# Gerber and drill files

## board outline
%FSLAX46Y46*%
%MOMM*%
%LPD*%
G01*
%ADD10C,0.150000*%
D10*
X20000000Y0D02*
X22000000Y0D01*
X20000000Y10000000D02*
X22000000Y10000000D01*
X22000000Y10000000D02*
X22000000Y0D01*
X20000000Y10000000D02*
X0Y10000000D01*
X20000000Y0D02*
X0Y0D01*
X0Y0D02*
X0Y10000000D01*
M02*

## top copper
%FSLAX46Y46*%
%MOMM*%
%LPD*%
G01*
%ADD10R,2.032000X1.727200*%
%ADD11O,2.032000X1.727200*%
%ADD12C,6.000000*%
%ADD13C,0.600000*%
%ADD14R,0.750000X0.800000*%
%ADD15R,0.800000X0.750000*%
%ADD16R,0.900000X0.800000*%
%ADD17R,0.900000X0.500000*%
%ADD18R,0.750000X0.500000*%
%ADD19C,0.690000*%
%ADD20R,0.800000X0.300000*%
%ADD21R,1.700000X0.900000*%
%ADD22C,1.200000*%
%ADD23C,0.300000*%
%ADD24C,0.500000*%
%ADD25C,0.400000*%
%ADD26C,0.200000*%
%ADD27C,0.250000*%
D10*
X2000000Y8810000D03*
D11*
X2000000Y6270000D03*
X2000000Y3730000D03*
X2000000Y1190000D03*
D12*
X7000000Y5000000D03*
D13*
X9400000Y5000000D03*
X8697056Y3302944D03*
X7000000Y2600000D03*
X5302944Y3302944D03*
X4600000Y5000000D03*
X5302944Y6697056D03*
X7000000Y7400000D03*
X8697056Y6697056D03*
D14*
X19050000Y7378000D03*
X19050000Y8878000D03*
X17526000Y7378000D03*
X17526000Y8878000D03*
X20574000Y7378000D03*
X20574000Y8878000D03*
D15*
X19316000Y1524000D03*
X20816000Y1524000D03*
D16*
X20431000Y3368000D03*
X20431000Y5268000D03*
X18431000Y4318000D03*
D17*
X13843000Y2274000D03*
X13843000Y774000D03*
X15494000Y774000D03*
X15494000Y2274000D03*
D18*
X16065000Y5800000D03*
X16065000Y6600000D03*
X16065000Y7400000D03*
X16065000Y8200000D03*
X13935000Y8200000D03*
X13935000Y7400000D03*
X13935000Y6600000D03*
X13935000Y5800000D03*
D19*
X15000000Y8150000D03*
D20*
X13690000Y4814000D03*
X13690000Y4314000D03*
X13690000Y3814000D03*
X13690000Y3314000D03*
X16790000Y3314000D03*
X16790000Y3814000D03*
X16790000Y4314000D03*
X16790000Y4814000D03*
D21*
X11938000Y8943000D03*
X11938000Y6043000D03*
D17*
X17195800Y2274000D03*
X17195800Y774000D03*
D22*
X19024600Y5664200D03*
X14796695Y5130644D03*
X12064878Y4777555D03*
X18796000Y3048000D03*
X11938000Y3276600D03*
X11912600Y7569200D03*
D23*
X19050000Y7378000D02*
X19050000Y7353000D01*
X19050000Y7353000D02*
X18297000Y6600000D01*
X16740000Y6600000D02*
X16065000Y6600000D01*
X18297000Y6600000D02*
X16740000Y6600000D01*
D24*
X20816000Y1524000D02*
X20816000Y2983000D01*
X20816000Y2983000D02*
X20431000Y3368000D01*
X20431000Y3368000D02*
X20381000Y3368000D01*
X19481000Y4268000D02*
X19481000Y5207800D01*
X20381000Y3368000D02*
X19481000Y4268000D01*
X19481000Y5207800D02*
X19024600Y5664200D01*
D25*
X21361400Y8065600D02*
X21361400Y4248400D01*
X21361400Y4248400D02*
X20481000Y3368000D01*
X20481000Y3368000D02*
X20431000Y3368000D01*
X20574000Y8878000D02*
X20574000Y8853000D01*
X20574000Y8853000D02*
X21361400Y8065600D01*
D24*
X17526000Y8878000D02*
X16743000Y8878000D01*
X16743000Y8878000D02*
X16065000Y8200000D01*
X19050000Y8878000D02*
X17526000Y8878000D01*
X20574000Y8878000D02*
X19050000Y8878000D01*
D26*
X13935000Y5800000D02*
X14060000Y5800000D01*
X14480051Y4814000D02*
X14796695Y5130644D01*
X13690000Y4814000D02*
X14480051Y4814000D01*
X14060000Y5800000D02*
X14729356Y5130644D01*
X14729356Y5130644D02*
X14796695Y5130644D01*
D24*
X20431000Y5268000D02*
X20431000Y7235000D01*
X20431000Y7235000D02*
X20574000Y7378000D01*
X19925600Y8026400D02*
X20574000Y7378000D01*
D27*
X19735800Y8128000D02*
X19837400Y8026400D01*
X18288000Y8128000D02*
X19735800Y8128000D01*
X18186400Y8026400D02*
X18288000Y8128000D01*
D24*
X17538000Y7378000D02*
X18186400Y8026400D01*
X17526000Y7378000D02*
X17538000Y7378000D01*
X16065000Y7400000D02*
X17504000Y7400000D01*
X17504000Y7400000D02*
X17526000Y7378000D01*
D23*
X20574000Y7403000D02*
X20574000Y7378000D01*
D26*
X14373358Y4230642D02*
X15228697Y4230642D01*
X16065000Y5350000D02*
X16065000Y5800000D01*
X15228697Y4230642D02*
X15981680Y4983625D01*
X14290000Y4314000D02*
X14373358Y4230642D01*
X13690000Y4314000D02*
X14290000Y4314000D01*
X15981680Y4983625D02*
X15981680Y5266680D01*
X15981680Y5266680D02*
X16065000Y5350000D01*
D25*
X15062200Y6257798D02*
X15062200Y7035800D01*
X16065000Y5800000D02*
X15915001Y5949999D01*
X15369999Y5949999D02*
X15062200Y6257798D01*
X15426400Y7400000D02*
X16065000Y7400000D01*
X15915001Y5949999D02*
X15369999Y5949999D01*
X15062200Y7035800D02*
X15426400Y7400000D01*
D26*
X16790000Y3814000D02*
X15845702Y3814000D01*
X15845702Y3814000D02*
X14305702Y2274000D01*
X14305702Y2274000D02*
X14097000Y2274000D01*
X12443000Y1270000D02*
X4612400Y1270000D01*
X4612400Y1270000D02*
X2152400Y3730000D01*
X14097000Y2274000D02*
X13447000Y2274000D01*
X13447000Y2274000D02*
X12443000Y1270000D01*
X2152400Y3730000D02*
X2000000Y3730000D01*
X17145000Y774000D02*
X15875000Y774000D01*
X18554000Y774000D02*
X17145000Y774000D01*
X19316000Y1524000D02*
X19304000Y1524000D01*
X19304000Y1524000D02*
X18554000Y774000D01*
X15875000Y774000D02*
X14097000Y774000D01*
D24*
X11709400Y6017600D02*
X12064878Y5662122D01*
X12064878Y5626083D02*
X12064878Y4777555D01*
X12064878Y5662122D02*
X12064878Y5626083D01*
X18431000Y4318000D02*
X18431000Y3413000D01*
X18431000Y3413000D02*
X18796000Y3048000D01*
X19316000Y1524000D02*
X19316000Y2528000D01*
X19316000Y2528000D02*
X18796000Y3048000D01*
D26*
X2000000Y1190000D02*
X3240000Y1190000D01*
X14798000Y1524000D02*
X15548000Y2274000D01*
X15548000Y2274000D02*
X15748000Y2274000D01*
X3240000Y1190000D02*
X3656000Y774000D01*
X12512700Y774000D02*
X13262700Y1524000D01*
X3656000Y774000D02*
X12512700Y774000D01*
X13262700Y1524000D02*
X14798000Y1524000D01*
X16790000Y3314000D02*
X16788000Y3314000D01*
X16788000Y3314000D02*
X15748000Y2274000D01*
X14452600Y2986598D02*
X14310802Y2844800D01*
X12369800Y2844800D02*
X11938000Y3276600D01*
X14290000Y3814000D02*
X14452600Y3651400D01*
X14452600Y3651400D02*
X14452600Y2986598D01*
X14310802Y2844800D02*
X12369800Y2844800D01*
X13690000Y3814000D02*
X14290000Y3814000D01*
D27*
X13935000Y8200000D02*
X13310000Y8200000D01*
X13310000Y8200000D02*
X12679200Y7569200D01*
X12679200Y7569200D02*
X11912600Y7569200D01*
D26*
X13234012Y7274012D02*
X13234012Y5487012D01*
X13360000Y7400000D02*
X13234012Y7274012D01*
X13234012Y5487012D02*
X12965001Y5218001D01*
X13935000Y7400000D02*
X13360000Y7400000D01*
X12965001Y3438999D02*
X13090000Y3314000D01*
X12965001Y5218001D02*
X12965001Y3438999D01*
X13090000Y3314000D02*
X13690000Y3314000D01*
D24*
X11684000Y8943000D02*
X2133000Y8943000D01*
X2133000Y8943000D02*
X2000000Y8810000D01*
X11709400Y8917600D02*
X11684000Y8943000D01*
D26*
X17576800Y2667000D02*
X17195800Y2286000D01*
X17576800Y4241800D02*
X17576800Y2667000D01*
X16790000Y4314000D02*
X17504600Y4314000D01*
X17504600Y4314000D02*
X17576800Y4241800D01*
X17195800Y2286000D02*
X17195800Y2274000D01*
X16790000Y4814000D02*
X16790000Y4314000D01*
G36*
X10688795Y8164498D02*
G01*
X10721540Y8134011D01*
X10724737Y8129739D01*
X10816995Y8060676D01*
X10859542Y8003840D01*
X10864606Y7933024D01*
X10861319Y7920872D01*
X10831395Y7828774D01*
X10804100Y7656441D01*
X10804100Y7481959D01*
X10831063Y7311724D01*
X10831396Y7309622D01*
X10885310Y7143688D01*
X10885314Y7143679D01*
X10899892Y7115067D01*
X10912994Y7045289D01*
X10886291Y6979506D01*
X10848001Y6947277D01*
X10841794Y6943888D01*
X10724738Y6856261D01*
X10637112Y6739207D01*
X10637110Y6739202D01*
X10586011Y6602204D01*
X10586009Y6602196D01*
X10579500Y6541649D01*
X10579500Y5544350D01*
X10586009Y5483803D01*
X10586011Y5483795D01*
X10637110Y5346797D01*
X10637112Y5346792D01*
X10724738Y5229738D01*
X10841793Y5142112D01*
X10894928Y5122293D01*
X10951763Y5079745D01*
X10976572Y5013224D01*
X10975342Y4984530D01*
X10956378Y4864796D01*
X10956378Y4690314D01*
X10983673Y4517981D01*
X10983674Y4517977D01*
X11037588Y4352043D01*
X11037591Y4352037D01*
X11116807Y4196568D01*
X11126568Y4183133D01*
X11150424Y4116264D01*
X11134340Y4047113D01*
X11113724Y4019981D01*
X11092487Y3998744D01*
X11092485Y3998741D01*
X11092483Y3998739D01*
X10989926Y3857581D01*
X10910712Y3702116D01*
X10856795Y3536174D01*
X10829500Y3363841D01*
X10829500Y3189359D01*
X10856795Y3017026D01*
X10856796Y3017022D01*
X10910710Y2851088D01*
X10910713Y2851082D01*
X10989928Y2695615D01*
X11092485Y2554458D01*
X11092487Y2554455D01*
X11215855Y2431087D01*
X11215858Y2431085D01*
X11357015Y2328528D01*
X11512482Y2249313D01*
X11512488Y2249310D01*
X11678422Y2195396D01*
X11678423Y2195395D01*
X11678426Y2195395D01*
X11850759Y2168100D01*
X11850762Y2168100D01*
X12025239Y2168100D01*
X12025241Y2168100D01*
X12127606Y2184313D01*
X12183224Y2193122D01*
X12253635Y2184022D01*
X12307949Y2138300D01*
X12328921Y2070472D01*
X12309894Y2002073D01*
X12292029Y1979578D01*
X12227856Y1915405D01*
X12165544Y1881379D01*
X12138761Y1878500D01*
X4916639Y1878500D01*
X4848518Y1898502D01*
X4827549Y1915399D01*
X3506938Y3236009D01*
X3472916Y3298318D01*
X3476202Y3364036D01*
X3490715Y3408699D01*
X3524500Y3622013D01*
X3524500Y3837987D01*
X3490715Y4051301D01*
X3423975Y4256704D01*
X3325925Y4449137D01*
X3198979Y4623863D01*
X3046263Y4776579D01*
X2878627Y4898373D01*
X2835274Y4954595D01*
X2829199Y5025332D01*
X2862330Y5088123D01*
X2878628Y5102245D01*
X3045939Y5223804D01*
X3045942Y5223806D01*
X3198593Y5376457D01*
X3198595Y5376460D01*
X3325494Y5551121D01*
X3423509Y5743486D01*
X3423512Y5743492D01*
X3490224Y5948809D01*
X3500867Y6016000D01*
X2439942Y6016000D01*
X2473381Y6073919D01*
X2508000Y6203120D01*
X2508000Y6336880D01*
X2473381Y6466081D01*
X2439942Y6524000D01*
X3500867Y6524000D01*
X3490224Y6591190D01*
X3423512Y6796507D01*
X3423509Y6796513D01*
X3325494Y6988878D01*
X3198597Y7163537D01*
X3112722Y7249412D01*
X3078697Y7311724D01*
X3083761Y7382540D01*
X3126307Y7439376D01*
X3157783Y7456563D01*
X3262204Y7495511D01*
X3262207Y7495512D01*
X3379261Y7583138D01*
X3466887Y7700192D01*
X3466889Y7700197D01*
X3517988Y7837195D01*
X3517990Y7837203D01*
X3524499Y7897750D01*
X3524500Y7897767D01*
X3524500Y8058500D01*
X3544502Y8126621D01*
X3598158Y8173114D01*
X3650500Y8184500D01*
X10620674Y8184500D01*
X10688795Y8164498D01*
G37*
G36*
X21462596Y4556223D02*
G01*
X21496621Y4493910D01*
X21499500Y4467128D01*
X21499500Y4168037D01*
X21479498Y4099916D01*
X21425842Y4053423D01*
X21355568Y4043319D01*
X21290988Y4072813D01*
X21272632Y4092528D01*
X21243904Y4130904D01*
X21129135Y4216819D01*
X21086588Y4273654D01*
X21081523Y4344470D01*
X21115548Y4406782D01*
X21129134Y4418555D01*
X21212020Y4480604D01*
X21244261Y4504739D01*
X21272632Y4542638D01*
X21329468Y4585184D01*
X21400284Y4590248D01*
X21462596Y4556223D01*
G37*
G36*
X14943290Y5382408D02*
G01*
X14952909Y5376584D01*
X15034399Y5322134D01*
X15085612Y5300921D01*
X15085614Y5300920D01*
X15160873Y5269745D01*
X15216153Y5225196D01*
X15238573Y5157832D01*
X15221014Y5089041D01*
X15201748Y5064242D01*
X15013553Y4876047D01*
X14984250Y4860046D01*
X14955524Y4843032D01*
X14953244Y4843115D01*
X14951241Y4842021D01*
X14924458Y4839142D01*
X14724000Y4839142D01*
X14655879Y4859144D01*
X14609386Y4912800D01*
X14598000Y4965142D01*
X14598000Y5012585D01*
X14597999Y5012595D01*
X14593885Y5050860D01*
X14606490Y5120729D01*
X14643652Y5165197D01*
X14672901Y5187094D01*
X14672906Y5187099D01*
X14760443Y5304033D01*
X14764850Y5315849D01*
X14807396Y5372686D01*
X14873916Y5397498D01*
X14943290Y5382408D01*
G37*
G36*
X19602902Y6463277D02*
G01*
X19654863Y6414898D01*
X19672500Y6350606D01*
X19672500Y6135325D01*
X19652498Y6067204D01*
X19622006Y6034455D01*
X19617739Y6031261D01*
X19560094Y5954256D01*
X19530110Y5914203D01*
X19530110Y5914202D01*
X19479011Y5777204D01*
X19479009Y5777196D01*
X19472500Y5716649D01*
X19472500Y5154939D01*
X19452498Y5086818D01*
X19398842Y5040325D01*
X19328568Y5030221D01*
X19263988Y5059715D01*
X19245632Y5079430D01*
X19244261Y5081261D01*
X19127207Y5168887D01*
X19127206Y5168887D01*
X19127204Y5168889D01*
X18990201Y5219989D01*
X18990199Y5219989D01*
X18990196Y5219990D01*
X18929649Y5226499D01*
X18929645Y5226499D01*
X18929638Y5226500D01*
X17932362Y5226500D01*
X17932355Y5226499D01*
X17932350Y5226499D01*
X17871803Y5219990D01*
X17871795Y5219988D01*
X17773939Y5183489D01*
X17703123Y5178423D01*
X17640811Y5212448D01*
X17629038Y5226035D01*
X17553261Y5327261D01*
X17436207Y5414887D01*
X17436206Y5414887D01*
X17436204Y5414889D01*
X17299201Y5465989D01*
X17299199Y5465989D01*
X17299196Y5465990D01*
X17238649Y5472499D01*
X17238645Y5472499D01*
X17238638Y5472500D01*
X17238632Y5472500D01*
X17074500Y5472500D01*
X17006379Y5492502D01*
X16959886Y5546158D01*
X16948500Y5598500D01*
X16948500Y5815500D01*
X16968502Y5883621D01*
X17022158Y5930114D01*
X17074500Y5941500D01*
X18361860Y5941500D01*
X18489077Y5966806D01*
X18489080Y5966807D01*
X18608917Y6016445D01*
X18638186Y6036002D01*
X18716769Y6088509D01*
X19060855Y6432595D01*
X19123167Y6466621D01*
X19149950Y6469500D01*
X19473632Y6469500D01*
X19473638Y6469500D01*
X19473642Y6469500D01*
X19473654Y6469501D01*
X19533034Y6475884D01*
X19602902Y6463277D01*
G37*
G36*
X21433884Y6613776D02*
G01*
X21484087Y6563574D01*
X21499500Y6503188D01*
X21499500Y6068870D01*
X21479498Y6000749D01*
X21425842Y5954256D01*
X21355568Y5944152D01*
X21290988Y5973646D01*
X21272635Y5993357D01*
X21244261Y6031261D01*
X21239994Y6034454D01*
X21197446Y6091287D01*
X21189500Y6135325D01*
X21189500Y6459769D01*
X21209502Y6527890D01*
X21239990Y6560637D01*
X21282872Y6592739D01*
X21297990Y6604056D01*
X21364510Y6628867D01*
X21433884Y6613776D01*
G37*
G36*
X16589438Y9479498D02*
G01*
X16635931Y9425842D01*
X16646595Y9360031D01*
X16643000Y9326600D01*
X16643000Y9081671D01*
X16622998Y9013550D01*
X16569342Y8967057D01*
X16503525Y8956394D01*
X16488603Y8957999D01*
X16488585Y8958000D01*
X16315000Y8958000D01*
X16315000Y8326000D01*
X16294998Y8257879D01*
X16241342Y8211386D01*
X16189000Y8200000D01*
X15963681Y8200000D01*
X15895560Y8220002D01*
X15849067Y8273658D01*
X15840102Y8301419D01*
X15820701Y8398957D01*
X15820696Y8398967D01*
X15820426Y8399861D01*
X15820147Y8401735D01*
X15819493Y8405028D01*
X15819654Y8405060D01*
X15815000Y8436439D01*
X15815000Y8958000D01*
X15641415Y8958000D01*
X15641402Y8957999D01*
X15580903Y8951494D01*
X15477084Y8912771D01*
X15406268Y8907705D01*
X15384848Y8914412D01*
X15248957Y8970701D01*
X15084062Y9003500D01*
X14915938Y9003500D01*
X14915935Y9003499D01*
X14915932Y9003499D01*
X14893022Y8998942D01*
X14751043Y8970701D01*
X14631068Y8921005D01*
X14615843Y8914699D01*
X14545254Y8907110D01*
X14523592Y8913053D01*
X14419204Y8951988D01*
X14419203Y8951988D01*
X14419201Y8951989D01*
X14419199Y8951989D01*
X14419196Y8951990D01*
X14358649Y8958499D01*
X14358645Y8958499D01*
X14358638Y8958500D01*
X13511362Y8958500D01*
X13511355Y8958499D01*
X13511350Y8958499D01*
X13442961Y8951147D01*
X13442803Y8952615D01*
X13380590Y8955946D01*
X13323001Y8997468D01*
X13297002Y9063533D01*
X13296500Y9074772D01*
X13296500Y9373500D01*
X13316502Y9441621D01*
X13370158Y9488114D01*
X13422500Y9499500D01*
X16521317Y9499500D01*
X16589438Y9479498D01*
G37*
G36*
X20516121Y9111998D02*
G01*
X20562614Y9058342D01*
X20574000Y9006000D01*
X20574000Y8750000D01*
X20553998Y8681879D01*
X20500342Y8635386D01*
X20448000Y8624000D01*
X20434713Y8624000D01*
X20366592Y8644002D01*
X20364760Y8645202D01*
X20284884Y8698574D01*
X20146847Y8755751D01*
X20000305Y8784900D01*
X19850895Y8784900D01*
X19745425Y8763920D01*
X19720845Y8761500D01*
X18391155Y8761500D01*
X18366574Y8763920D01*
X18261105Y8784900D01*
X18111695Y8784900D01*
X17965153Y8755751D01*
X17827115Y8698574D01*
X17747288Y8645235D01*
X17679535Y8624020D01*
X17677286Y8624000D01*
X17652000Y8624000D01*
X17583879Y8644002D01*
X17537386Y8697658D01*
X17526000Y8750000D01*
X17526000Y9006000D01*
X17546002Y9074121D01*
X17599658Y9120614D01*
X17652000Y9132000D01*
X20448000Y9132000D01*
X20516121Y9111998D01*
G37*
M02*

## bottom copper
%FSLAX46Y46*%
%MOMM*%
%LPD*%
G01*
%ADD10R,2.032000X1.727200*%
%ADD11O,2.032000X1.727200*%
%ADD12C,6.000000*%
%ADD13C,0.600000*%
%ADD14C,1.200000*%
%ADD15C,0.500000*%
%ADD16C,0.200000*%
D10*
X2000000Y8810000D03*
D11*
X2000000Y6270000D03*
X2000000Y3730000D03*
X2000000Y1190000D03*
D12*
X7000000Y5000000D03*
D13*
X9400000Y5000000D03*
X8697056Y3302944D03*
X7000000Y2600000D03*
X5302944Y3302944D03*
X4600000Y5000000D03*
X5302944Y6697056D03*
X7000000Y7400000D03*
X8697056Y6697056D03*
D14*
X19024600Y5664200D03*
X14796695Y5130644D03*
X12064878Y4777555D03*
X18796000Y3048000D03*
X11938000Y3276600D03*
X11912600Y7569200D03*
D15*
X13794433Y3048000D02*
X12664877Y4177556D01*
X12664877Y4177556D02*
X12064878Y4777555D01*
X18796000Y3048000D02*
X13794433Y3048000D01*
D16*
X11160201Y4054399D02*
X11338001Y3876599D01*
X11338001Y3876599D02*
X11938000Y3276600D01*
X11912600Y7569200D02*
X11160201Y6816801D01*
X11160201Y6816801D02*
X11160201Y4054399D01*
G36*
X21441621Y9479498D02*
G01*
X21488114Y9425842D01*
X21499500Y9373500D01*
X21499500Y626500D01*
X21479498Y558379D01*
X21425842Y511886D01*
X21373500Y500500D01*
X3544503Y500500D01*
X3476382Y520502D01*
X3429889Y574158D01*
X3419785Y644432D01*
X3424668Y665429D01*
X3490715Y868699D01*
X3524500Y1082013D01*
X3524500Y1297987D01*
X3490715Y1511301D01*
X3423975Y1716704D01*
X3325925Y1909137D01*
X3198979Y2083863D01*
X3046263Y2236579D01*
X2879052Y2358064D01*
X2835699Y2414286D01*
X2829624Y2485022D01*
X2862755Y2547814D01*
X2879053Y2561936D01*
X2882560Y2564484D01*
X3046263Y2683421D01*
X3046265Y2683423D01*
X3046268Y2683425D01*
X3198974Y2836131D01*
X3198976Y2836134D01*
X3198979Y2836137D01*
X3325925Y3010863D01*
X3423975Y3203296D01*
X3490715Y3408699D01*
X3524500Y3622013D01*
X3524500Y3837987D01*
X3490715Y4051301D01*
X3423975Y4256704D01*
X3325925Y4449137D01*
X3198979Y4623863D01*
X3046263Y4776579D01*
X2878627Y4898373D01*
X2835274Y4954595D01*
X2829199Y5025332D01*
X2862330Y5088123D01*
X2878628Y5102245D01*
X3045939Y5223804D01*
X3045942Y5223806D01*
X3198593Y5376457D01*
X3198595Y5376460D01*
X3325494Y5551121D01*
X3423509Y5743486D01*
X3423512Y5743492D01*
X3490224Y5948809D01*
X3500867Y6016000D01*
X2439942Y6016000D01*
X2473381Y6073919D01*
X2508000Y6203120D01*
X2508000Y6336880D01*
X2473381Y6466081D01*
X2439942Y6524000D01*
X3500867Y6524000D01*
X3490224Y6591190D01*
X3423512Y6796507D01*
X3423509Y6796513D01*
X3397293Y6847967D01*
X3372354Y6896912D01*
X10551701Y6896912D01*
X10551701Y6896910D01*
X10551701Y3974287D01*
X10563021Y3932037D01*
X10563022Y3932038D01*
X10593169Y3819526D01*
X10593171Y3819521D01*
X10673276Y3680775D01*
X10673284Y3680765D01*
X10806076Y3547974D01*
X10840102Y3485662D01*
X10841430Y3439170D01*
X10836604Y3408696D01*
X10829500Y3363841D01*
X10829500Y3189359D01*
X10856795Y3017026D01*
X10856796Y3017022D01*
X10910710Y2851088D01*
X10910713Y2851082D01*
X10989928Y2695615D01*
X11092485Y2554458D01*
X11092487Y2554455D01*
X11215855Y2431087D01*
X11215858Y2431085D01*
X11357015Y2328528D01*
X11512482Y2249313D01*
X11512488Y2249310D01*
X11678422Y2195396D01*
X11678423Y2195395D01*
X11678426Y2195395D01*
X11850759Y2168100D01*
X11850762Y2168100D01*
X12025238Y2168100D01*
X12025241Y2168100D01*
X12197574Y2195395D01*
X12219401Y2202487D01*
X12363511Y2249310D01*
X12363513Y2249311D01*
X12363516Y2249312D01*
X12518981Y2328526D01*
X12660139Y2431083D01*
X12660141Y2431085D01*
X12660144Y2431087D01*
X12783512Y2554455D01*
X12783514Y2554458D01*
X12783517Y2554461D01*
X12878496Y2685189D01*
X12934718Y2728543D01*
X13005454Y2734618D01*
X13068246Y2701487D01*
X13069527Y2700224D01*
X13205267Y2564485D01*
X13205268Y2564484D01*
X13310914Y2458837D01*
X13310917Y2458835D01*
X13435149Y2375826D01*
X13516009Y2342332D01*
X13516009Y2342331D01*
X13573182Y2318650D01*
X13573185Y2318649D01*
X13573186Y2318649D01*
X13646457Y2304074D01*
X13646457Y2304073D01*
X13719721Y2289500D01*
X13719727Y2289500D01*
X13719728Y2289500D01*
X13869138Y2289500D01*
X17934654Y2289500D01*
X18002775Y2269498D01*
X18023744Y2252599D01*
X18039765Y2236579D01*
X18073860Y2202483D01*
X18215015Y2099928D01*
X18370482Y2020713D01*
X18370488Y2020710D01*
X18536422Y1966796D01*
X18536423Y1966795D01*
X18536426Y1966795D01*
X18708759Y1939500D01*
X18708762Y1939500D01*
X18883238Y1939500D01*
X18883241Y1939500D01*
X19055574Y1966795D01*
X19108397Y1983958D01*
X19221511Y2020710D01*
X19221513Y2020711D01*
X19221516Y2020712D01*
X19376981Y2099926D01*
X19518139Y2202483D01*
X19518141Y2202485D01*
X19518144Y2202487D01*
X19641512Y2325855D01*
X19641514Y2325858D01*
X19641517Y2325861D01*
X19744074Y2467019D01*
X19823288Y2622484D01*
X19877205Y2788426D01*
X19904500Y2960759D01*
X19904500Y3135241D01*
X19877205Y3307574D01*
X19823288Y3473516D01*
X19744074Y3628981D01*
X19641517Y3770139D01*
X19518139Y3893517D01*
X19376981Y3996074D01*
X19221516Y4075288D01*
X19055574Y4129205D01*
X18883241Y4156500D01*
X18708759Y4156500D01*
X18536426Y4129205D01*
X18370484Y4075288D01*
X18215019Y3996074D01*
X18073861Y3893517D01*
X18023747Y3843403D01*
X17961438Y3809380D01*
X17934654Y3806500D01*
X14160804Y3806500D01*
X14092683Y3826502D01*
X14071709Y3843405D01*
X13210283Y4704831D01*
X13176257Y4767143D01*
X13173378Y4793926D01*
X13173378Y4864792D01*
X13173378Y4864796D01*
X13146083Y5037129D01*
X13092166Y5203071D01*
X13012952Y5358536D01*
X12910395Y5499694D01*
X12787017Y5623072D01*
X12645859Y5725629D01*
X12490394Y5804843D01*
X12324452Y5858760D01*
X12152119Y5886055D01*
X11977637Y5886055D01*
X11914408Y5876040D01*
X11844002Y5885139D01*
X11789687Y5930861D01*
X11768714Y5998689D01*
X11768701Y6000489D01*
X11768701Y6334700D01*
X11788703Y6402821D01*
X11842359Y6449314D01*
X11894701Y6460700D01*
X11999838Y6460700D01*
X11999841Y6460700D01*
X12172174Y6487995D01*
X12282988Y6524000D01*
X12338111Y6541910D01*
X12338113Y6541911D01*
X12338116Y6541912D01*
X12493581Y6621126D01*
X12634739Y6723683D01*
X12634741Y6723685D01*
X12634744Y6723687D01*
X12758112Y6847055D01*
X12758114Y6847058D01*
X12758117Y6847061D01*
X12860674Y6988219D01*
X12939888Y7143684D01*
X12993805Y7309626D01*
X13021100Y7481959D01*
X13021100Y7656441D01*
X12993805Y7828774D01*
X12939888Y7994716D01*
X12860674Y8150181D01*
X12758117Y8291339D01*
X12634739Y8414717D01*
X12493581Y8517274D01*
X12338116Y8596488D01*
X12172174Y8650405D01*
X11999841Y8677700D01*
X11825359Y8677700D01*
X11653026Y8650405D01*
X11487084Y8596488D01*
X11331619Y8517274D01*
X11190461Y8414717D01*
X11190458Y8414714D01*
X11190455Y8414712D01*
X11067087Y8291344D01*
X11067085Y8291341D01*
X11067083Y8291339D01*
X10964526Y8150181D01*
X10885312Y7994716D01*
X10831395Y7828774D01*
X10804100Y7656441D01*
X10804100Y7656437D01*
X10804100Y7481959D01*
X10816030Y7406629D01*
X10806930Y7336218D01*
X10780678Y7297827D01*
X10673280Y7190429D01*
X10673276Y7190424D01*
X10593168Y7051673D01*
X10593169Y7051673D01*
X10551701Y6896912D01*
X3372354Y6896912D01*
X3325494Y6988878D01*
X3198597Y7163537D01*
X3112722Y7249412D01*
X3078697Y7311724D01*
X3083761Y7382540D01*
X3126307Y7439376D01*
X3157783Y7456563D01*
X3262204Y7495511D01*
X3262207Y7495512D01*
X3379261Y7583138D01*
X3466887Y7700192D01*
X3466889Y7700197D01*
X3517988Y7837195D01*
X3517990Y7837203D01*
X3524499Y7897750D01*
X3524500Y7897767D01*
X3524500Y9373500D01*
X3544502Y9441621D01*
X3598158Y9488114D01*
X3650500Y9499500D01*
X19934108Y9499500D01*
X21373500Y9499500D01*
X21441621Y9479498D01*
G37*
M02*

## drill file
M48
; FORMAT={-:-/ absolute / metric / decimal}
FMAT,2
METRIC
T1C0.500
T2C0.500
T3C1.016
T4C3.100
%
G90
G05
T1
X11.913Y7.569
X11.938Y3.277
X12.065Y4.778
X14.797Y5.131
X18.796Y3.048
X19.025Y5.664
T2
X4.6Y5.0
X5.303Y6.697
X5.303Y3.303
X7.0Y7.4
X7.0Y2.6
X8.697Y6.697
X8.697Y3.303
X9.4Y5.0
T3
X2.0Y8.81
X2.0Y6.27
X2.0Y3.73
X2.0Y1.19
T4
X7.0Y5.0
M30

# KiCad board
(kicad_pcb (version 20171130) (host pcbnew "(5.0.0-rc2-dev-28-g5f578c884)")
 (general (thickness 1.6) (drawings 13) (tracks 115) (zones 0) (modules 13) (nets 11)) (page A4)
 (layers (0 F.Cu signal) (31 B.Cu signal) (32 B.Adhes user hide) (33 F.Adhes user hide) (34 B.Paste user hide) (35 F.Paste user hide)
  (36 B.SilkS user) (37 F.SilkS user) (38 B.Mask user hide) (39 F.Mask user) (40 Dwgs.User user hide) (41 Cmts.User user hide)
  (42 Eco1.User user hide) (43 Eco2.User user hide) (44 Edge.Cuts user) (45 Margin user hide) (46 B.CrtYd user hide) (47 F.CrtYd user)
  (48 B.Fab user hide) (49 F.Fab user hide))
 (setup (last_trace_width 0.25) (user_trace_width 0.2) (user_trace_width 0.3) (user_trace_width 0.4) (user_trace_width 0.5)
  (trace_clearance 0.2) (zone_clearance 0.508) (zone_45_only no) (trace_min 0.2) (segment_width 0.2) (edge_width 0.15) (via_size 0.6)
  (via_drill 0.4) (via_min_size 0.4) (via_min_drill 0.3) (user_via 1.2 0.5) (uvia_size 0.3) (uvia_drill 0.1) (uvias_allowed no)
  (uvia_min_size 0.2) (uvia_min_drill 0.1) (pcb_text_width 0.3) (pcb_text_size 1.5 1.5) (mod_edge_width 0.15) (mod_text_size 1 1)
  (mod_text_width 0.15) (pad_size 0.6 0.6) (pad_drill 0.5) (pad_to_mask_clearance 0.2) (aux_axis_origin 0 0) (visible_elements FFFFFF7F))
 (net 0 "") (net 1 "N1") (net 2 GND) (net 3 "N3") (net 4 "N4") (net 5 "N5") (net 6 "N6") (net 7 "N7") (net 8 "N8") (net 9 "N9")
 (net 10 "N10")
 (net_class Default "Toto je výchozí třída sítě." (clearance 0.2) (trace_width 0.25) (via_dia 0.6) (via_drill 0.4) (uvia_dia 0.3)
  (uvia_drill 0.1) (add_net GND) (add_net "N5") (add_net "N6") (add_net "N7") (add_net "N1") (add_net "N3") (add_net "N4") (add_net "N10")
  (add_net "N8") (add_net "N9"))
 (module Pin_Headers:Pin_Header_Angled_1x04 (layer B.Cu) (at 2 -8.81 180)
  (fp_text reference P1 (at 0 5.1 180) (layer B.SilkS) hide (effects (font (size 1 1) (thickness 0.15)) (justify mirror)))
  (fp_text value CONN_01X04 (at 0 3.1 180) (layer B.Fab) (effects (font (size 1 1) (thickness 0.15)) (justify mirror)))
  (pad 1 thru_hole rect (at 0 0 180) (size 2.032 1.7272) (drill 1.016) (layers *.Cu *.Mask) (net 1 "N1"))
  (pad 2 thru_hole oval (at 0 -2.54 180) (size 2.032 1.7272) (drill 1.016) (layers *.Cu *.Mask) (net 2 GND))
  (pad 3 thru_hole oval (at 0 -5.08 180) (size 2.032 1.7272) (drill 1.016) (layers *.Cu *.Mask) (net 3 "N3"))
  (pad 4 thru_hole oval (at 0 -7.62 180) (size 2.032 1.7272) (drill 1.016) (layers *.Cu *.Mask) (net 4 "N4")))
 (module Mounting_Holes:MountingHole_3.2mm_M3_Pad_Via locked (layer F.Cu) (at 7 -5)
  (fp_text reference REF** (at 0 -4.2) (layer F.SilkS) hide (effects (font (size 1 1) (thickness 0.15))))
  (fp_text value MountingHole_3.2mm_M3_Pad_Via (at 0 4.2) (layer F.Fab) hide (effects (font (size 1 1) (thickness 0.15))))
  (pad 1 thru_hole circle (at 0 0) (size 6 6) (drill 3.1) (layers *.Cu *.Mask) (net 2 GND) (zone_connect 2))
  (pad "" thru_hole circle (at 2.4 0) (size 0.6 0.6) (drill 0.5) (layers *.Cu *.Mask) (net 2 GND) (zone_connect 2))
  (pad "" thru_hole circle (at 1.697056 1.697056) (size 0.6 0.6) (drill 0.5) (layers *.Cu *.Mask) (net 2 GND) (zone_connect 2))
  (pad "" thru_hole circle (at 0 2.4) (size 0.6 0.6) (drill 0.5) (layers *.Cu *.Mask) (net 2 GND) (zone_connect 2))
  (pad "" thru_hole circle (at -1.697056 1.697056) (size 0.6 0.6) (drill 0.5) (layers *.Cu *.Mask) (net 2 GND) (zone_connect 2))
  (pad "" thru_hole circle (at -2.4 0) (size 0.6 0.6) (drill 0.5) (layers *.Cu *.Mask) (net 2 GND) (zone_connect 2))
  (pad "" thru_hole circle (at -1.697056 -1.697056) (size 0.6 0.6) (drill 0.5) (layers *.Cu *.Mask) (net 2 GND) (zone_connect 2))
  (pad "" thru_hole circle (at 0 -2.4) (size 0.6 0.6) (drill 0.5) (layers *.Cu *.Mask) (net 2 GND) (zone_connect 2))
  (pad "" thru_hole circle (at 1.697056 -1.697056) (size 0.6 0.6) (drill 0.5) (layers *.Cu *.Mask) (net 2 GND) (zone_connect 2)))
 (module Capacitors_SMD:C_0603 (layer F.Cu) (at 19.05 -8.128 90)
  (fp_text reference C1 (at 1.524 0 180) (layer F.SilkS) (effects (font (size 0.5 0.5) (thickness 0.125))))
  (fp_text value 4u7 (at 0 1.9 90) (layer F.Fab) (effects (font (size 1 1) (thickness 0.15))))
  (pad 1 smd rect (at -0.75 0 90) (size 0.8 0.75) (layers F.Cu F.Paste F.Mask) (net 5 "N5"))
  (pad 2 smd rect (at 0.75 0 90) (size 0.8 0.75) (layers F.Cu F.Paste F.Mask) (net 2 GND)))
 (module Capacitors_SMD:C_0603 (layer F.Cu) (at 17.526 -8.128 90)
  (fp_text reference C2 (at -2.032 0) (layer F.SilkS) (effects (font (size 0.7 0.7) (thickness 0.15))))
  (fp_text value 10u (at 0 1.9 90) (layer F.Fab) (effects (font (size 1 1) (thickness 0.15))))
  (pad 1 smd rect (at -0.75 0 90) (size 0.8 0.75) (layers F.Cu F.Paste F.Mask) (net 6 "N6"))
  (pad 2 smd rect (at 0.75 0 90) (size 0.8 0.75) (layers F.Cu F.Paste F.Mask) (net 2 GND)))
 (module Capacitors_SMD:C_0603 (layer F.Cu) (at 20.574 -8.128 90)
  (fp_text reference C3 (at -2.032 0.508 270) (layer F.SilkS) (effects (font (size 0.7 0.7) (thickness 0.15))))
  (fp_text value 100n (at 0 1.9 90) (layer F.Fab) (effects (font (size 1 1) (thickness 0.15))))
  (pad 1 smd rect (at -0.75 0 90) (size 0.8 0.75) (layers F.Cu F.Paste F.Mask) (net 6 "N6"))
  (pad 2 smd rect (at 0.75 0 90) (size 0.8 0.75) (layers F.Cu F.Paste F.Mask) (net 2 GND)))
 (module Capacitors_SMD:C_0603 (layer F.Cu) (at 20.066 -1.524)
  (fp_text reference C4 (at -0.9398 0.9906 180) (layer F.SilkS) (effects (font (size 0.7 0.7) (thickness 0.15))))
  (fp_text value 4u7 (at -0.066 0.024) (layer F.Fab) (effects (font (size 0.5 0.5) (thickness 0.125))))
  (pad 1 smd rect (at -0.75 0) (size 0.8 0.75) (layers F.Cu F.Paste F.Mask) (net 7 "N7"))
  (pad 2 smd rect (at 0.75 0) (size 0.8 0.75) (layers F.Cu F.Paste F.Mask) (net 2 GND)))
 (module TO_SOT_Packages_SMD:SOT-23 (layer F.Cu) (at 19.431 -4.318 180)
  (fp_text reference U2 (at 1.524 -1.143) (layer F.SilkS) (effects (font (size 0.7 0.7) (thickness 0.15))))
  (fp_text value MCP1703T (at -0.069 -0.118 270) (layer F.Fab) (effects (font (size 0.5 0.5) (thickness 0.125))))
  (pad 1 smd rect (at -1 -0.95 180) (size 0.9 0.8) (layers F.Cu F.Paste F.Mask) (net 2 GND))
  (pad 2 smd rect (at -1 0.95 180) (size 0.9 0.8) (layers F.Cu F.Paste F.Mask) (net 6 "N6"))
  (pad 3 smd rect (at 1 0 180) (size 0.9 0.8) (layers F.Cu F.Paste F.Mask) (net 7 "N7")))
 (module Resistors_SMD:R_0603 (layer F.Cu) (at 13.843 -1.524 270)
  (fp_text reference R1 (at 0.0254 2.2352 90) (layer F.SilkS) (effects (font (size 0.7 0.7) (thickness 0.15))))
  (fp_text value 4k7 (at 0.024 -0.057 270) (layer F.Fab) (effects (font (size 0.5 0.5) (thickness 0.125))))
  (pad 1 smd rect (at -0.75 0 270) (size 0.5 0.9) (layers F.Cu F.Paste F.Mask) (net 3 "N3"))
  (pad 2 smd rect (at 0.75 0 270) (size 0.5 0.9) (layers F.Cu F.Paste F.Mask) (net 7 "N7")))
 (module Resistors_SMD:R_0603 (layer F.Cu) (at 15.494 -1.524 90)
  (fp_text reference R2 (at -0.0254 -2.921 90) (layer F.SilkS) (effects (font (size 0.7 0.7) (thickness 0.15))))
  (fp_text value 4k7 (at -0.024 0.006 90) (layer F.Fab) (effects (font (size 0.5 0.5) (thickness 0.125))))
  (pad 1 smd rect (at -0.75 0 90) (size 0.5 0.9) (layers F.Cu F.Paste F.Mask) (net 7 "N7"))
  (pad 2 smd rect (at 0.75 0 90) (size 0.5 0.9) (layers F.Cu F.Paste F.Mask) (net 4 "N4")))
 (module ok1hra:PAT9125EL (layer F.Cu) (at 15 -7 90)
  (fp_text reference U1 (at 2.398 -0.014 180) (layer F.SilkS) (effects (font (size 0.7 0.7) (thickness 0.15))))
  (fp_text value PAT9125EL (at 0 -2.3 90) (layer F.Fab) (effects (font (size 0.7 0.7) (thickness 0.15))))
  (pad 1 smd rect (at -1.2 1.065 90) (size 0.5 0.75) (layers F.Cu F.Paste F.Mask) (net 6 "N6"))
  (pad 2 smd rect (at -0.4 1.065 90) (size 0.5 0.75) (layers F.Cu F.Paste F.Mask) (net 5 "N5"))
  (pad 3 smd rect (at 0.4 1.065 90) (size 0.5 0.75) (layers F.Cu F.Paste F.Mask) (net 6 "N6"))
  (pad 4 smd rect (at 1.2 1.065 90) (size 0.5 0.75) (layers F.Cu F.Paste F.Mask) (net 2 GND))
  (pad 5 smd rect (at 1.2 -1.065 90) (size 0.5 0.75) (layers F.Cu F.Paste F.Mask) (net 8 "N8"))
  (pad 6 smd rect (at 0.4 -1.065 90) (size 0.5 0.75) (layers F.Cu F.Paste F.Mask) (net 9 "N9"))
  (pad 7 smd rect (at -0.4 -1.065 90) (size 0.5 0.75) (layers F.Cu F.Paste F.Mask))
  (pad 8 smd rect (at -1.2 -1.065 90) (size 0.5 0.75) (layers F.Cu F.Paste F.Mask) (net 2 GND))
  (pad 9 smd circle (at 1.15 0 90) (size 0.69 0.69) (layers F.Cu F.Paste F.Mask)))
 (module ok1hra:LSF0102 (layer F.Cu) (at 15.24 -4.064 90)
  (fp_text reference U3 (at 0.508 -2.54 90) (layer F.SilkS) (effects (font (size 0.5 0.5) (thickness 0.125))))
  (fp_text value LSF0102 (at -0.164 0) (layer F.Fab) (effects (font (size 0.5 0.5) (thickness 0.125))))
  (pad 1 smd rect (at 0.75 -1.55 270) (size 0.3 0.8) (layers F.Cu F.Paste F.Mask) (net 2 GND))
  (pad 2 smd rect (at 0.25 -1.55 270) (size 0.3 0.8) (layers F.Cu F.Paste F.Mask) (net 6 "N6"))
  (pad 3 smd rect (at -0.25 -1.55 270) (size 0.3 0.8) (layers F.Cu F.Paste F.Mask) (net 8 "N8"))
  (pad 4 smd rect (at -0.75 -1.55 270) (size 0.3 0.8) (layers F.Cu F.Paste F.Mask) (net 9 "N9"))
  (pad 5 smd rect (at -0.75 1.55 270) (size 0.3 0.8) (layers F.Cu F.Paste F.Mask) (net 4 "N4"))
  (pad 6 smd rect (at -0.25 1.55 270) (size 0.3 0.8) (layers F.Cu F.Paste F.Mask) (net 3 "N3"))
  (pad 7 smd rect (at 0.25 1.55 270) (size 0.3 0.8) (layers F.Cu F.Paste F.Mask) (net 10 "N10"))
  (pad 8 smd rect (at 0.75 1.55 270) (size 0.3 0.8) (layers F.Cu F.Paste F.Mask) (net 10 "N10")))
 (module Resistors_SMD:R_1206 (layer F.Cu) (at 11.938 -7.493 270)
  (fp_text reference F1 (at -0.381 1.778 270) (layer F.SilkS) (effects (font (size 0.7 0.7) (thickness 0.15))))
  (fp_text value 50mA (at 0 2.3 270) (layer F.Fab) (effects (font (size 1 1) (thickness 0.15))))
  (pad 1 smd rect (at -1.45 0 270) (size 0.9 1.7) (layers F.Cu F.Paste F.Mask) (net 1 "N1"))
  (pad 2 smd rect (at 1.45 0 270) (size 0.9 1.7) (layers F.Cu F.Paste F.Mask) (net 7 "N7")))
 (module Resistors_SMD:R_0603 (layer F.Cu) (at 17.1958 -1.524 270)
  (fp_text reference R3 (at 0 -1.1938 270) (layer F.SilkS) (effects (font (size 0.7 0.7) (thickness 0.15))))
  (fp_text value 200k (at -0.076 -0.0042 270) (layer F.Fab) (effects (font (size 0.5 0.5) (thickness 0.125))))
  (pad 1 smd rect (at -0.75 0 270) (size 0.5 0.9) (layers F.Cu F.Paste F.Mask) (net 10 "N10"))
  (pad 2 smd rect (at 0.75 0 270) (size 0.5 0.9) (layers F.Cu F.Paste F.Mask) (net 7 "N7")))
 (gr_line (start 20 0) (end 22 0) (layer Edge.Cuts) (width 0.15))
 (gr_line (start 20 -10) (end 22 -10) (layer Edge.Cuts) (width 0.15))
 (gr_line (start 22 -10) (end 22 0) (layer Edge.Cuts) (width 0.15))
 (gr_line (start 20 -10) (end 0 -10) (layer Edge.Cuts) (width 0.15))
 (gr_line (start 20 0) (end 0 0) (angle 90) (layer Edge.Cuts) (width 0.15))
 (gr_line (start 0 0) (end 0 -10) (angle 90) (layer Edge.Cuts) (width 0.15))
 (segment (start 19.05 -7.378) (end 19.05 -7.353) (width 0.3) (layer F.Cu) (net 5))
 (segment (start 19.05 -7.353) (end 18.297 -6.6) (width 0.3) (layer F.Cu) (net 5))
 (segment (start 16.74 -6.6) (end 16.065 -6.6) (width 0.3) (layer F.Cu) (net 5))
 (segment (start 18.297 -6.6) (end 16.74 -6.6) (width 0.3) (layer F.Cu) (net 5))
 (segment (start 20.816 -1.524) (end 20.816 -2.983) (width 0.5) (layer F.Cu) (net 2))
 (segment (start 20.816 -2.983) (end 20.431 -3.368) (width 0.5) (layer F.Cu) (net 2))
 (segment (start 20.431 -3.368) (end 20.381 -3.368) (width 0.5) (layer F.Cu) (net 2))
 (segment (start 19.481 -4.268) (end 19.481 -5.2078) (width 0.5) (layer F.Cu) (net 2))
 (via (at 19.0246 -5.6642) (size 1.2) (drill 0.5) (layers F.Cu B.Cu) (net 2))
 (segment (start 20.381 -3.368) (end 19.481 -4.268) (width 0.5) (layer F.Cu) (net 2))
 (segment (start 19.481 -5.2078) (end 19.0246 -5.6642) (width 0.5) (layer F.Cu) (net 2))
 (segment (start 21.3614 -8.0656) (end 21.3614 -4.2484) (width 0.4) (layer F.Cu) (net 2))
 (segment (start 21.3614 -4.2484) (end 20.481 -3.368) (width 0.4) (layer F.Cu) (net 2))
 (segment (start 20.481 -3.368) (end 20.431 -3.368) (width 0.4) (layer F.Cu) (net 2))
 (segment (start 20.574 -8.878) (end 20.574 -8.853) (width 0.4) (layer F.Cu) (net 2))
 (segment (start 20.574 -8.853) (end 21.3614 -8.0656) (width 0.4) (layer F.Cu) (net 2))
 (segment (start 17.526 -8.878) (end 16.743 -8.878) (width 0.5) (layer F.Cu) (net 2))
 (segment (start 16.743 -8.878) (end 16.065 -8.2) (width 0.5) (layer F.Cu) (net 2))
 (segment (start 19.05 -8.878) (end 17.526 -8.878) (width 0.5) (layer F.Cu) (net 2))
 (segment (start 20.574 -8.878) (end 19.05 -8.878) (width 0.5) (layer F.Cu) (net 2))
 (segment (start 13.935 -5.8) (end 14.06 -5.8) (width 0.2) (layer F.Cu) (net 2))
 (segment (start 14.480051 -4.814) (end 14.796695 -5.130644) (width 0.2) (layer F.Cu) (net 2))
 (via (at 14.796695 -5.130644) (size 1.2) (drill 0.5) (layers F.Cu B.Cu) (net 2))
 (segment (start 13.69 -4.814) (end 14.480051 -4.814) (width 0.2) (layer F.Cu) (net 2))
 (segment (start 14.06 -5.8) (end 14.729356 -5.130644) (width 0.2) (layer F.Cu) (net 2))
 (segment (start 14.729356 -5.130644) (end 14.796695 -5.130644) (width 0.2) (layer F.Cu) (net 2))
 (segment (start 20.431 -5.268) (end 20.431 -7.235) (width 0.5) (layer F.Cu) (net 6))
 (segment (start 20.431 -7.235) (end 20.574 -7.378) (width 0.5) (layer F.Cu) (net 6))
 (segment (start 19.9256 -8.0264) (end 20.574 -7.378) (width 0.5) (layer F.Cu) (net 6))
 (segment (start 19.7358 -8.128) (end 19.8374 -8.0264) (width 0.25) (layer F.Cu) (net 6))
 (segment (start 18.288 -8.128) (end 19.7358 -8.128) (width 0.25) (layer F.Cu) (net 6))
 (segment (start 18.1864 -8.0264) (end 18.288 -8.128) (width 0.25) (layer F.Cu) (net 6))
 (segment (start 17.538 -7.378) (end 18.1864 -8.0264) (width 0.5) (layer F.Cu) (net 6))
 (segment (start 17.526 -7.378) (end 17.538 -7.378) (width 0.5) (layer F.Cu) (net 6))
 (segment (start 16.065 -7.4) (end 17.504 -7.4) (width 0.5) (layer F.Cu) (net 6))
 (segment (start 17.504 -7.4) (end 17.526 -7.378) (width 0.5) (layer F.Cu) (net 6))
 (segment (start 20.574 -7.403) (end 20.574 -7.378) (width 0.3) (layer F.Cu) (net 6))
 (segment (start 14.373358 -4.230642) (end 15.228697 -4.230642) (width 0.2) (layer F.Cu) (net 6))
 (segment (start 16.065 -5.35) (end 16.065 -5.8) (width 0.2) (layer F.Cu) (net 6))
 (segment (start 15.228697 -4.230642) (end 15.98168 -4.983625) (width 0.2) (layer F.Cu) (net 6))
 (segment (start 14.29 -4.314) (end 14.373358 -4.230642) (width 0.2) (layer F.Cu) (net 6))
 (segment (start 13.69 -4.314) (end 14.29 -4.314) (width 0.2) (layer F.Cu) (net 6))
 (segment (start 15.98168 -4.983625) (end 15.98168 -5.26668) (width 0.2) (layer F.Cu) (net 6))
 (segment (start 15.98168 -5.26668) (end 16.065 -5.35) (width 0.2) (layer F.Cu) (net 6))
 (segment (start 15.0622 -6.257798) (end 15.0622 -7.0358) (width 0.4) (layer F.Cu) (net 6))
 (segment (start 16.065 -5.8) (end 15.915001 -5.949999) (width 0.4) (layer F.Cu) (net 6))
 (segment (start 15.369999 -5.949999) (end 15.0622 -6.257798) (width 0.4) (layer F.Cu) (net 6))
 (segment (start 15.4264 -7.4) (end 16.065 -7.4) (width 0.4) (layer F.Cu) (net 6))
 (segment (start 15.915001 -5.949999) (end 15.369999 -5.949999) (width 0.4) (layer F.Cu) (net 6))
 (segment (start 15.0622 -7.0358) (end 15.4264 -7.4) (width 0.4) (layer F.Cu) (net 6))
 (segment (start 16.79 -3.814) (end 15.845702 -3.814) (width 0.2) (layer F.Cu) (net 3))
 (segment (start 15.845702 -3.814) (end 14.305702 -2.274) (width 0.2) (layer F.Cu) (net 3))
 (segment (start 14.305702 -2.274) (end 14.097 -2.274) (width 0.2) (layer F.Cu) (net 3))
 (segment (start 12.443 -1.27) (end 4.6124 -1.27) (width 0.2) (layer F.Cu) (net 3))
 (segment (start 4.6124 -1.27) (end 2.1524 -3.73) (width 0.2) (layer F.Cu) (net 3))
 (segment (start 14.097 -2.274) (end 13.447 -2.274) (width 0.2) (layer F.Cu) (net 3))
 (segment (start 13.447 -2.274) (end 12.443 -1.27) (width 0.2) (layer F.Cu) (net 3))
 (segment (start 2.1524 -3.73) (end 2 -3.73) (width 0.2) (layer F.Cu) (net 3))
 (segment (start 17.145 -0.774) (end 15.875 -0.774) (width 0.2) (layer F.Cu) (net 7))
 (segment (start 18.554 -0.774) (end 17.145 -0.774) (width 0.2) (layer F.Cu) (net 7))
 (segment (start 19.316 -1.524) (end 19.304 -1.524) (width 0.2) (layer F.Cu) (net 7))
 (segment (start 19.304 -1.524) (end 18.554 -0.774) (width 0.2) (layer F.Cu) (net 7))
 (segment (start 15.875 -0.774) (end 14.097 -0.774) (width 0.2) (layer F.Cu) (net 7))
 (segment (start 13.794433 -3.048) (end 12.664877 -4.177556) (width 0.5) (layer B.Cu) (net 7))
 (segment (start 12.664877 -4.177556) (end 12.064878 -4.777555) (width 0.5) (layer B.Cu) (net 7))
 (segment (start 11.7094 -6.0176) (end 12.064878 -5.662122) (width 0.5) (layer F.Cu) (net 7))
 (segment (start 12.064878 -5.626083) (end 12.064878 -4.777555) (width 0.5) (layer F.Cu) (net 7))
 (segment (start 18.796 -3.048) (end 13.794433 -3.048) (width 0.5) (layer B.Cu) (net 7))
 (via (at 12.064878 -4.777555) (size 1.2) (drill 0.5) (layers F.Cu B.Cu) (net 7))
 (segment (start 12.064878 -5.662122) (end 12.064878 -5.626083) (width 0.5) (layer F.Cu) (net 7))
 (segment (start 18.431 -4.318) (end 18.431 -3.413) (width 0.5) (layer F.Cu) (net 7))
 (segment (start 18.431 -3.413) (end 18.796 -3.048) (width 0.5) (layer F.Cu) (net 7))
 (segment (start 19.316 -1.524) (end 19.316 -2.528) (width 0.5) (layer F.Cu) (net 7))
 (segment (start 19.316 -2.528) (end 18.796 -3.048) (width 0.5) (layer F.Cu) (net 7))
 (via (at 18.796 -3.048) (size 1.2) (drill 0.5) (layers F.Cu B.Cu) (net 7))
 (segment (start 2 -1.19) (end 3.24 -1.19) (width 0.2) (layer F.Cu) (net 4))
 (segment (start 14.798 -1.524) (end 15.548 -2.274) (width 0.2) (layer F.Cu) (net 4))
 (segment (start 15.548 -2.274) (end 15.748 -2.274) (width 0.2) (layer F.Cu) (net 4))
 (segment (start 3.24 -1.19) (end 3.656 -0.774) (width 0.2) (layer F.Cu) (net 4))
 (segment (start 12.5127 -0.774) (end 13.2627 -1.524) (width 0.2) (layer F.Cu) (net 4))
 (segment (start 3.656 -0.774) (end 12.5127 -0.774) (width 0.2) (layer F.Cu) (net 4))
 (segment (start 13.2627 -1.524) (end 14.798 -1.524) (width 0.2) (layer F.Cu) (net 4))
 (segment (start 16.79 -3.314) (end 16.788 -3.314) (width 0.2) (layer F.Cu) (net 4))
 (segment (start 16.788 -3.314) (end 15.748 -2.274) (width 0.2) (layer F.Cu) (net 4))
 (segment (start 14.4526 -2.986598) (end 14.310802 -2.8448) (width 0.2) (layer F.Cu) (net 8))
 (segment (start 12.3698 -2.8448) (end 11.938 -3.2766) (width 0.2) (layer F.Cu) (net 8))
 (segment (start 14.29 -3.814) (end 14.4526 -3.6514) (width 0.2) (layer F.Cu) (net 8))
 (segment (start 14.4526 -3.6514) (end 14.4526 -2.986598) (width 0.2) (layer F.Cu) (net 8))
 (segment (start 14.310802 -2.8448) (end 12.3698 -2.8448) (width 0.2) (layer F.Cu) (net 8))
 (segment (start 13.69 -3.814) (end 14.29 -3.814) (width 0.2) (layer F.Cu) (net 8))
 (segment (start 11.160201 -4.054399) (end 11.338001 -3.876599) (width 0.2) (layer B.Cu) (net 8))
 (segment (start 11.338001 -3.876599) (end 11.938 -3.2766) (width 0.2) (layer B.Cu) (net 8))
 (segment (start 11.9126 -7.5692) (end 11.160201 -6.816801) (width 0.2) (layer B.Cu) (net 8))
 (segment (start 11.160201 -6.816801) (end 11.160201 -4.054399) (width 0.2) (layer B.Cu) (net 8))
 (via (at 11.938 -3.2766) (size 1.2) (drill 0.5) (layers F.Cu B.Cu) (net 8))
 (segment (start 13.935 -8.2) (end 13.31 -8.2) (width 0.25) (layer F.Cu) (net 8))
 (segment (start 13.31 -8.2) (end 12.6792 -7.5692) (width 0.25) (layer F.Cu) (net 8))
 (via (at 11.9126 -7.5692) (size 1.2) (drill 0.5) (layers F.Cu B.Cu) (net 8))
 (segment (start 12.6792 -7.5692) (end 11.9126 -7.5692) (width 0.25) (layer F.Cu) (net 8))
 (segment (start 13.234012 -7.274012) (end 13.234012 -5.487012) (width 0.2) (layer F.Cu) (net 9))
 (segment (start 13.36 -7.4) (end 13.234012 -7.274012) (width 0.2) (layer F.Cu) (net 9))
 (segment (start 13.234012 -5.487012) (end 12.965001 -5.218001) (width 0.2) (layer F.Cu) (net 9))
 (segment (start 13.935 -7.4) (end 13.36 -7.4) (width 0.2) (layer F.Cu) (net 9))
 (segment (start 12.965001 -3.438999) (end 13.09 -3.314) (width 0.2) (layer F.Cu) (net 9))
 (segment (start 12.965001 -5.218001) (end 12.965001 -3.438999) (width 0.2) (layer F.Cu) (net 9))
 (segment (start 13.09 -3.314) (end 13.69 -3.314) (width 0.2) (layer F.Cu) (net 9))
 (segment (start 11.684 -8.943) (end 2.133 -8.943) (width 0.5) (layer F.Cu) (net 1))
 (segment (start 2.133 -8.943) (end 2 -8.81) (width 0.5) (layer F.Cu) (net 1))
 (segment (start 11.7094 -8.9176) (end 11.684 -8.943) (width 0.5) (layer F.Cu) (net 1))
 (segment (start 17.5768 -2.667) (end 17.1958 -2.286) (width 0.2) (layer F.Cu) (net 10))
 (segment (start 17.5768 -4.2418) (end 17.5768 -2.667) (width 0.2) (layer F.Cu) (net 10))
 (segment (start 16.79 -4.314) (end 17.5046 -4.314) (width 0.2) (layer F.Cu) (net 10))
 (segment (start 17.5046 -4.314) (end 17.5768 -4.2418) (width 0.2) (layer F.Cu) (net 10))
 (segment (start 17.1958 -2.286) (end 17.1958 -2.274) (width 0.2) (layer F.Cu) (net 10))
 (segment (start 16.79 -4.814) (end 16.79 -4.314) (width 0.2) (layer F.Cu) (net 10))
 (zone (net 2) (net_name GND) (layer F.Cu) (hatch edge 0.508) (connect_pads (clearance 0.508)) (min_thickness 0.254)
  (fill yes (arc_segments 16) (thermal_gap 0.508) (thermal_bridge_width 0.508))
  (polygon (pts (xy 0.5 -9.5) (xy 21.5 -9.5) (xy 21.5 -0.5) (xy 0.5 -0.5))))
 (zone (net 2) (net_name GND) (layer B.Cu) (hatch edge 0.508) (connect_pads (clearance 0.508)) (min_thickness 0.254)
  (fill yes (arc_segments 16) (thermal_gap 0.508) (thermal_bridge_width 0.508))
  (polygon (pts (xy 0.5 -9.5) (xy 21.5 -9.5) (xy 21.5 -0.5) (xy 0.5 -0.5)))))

